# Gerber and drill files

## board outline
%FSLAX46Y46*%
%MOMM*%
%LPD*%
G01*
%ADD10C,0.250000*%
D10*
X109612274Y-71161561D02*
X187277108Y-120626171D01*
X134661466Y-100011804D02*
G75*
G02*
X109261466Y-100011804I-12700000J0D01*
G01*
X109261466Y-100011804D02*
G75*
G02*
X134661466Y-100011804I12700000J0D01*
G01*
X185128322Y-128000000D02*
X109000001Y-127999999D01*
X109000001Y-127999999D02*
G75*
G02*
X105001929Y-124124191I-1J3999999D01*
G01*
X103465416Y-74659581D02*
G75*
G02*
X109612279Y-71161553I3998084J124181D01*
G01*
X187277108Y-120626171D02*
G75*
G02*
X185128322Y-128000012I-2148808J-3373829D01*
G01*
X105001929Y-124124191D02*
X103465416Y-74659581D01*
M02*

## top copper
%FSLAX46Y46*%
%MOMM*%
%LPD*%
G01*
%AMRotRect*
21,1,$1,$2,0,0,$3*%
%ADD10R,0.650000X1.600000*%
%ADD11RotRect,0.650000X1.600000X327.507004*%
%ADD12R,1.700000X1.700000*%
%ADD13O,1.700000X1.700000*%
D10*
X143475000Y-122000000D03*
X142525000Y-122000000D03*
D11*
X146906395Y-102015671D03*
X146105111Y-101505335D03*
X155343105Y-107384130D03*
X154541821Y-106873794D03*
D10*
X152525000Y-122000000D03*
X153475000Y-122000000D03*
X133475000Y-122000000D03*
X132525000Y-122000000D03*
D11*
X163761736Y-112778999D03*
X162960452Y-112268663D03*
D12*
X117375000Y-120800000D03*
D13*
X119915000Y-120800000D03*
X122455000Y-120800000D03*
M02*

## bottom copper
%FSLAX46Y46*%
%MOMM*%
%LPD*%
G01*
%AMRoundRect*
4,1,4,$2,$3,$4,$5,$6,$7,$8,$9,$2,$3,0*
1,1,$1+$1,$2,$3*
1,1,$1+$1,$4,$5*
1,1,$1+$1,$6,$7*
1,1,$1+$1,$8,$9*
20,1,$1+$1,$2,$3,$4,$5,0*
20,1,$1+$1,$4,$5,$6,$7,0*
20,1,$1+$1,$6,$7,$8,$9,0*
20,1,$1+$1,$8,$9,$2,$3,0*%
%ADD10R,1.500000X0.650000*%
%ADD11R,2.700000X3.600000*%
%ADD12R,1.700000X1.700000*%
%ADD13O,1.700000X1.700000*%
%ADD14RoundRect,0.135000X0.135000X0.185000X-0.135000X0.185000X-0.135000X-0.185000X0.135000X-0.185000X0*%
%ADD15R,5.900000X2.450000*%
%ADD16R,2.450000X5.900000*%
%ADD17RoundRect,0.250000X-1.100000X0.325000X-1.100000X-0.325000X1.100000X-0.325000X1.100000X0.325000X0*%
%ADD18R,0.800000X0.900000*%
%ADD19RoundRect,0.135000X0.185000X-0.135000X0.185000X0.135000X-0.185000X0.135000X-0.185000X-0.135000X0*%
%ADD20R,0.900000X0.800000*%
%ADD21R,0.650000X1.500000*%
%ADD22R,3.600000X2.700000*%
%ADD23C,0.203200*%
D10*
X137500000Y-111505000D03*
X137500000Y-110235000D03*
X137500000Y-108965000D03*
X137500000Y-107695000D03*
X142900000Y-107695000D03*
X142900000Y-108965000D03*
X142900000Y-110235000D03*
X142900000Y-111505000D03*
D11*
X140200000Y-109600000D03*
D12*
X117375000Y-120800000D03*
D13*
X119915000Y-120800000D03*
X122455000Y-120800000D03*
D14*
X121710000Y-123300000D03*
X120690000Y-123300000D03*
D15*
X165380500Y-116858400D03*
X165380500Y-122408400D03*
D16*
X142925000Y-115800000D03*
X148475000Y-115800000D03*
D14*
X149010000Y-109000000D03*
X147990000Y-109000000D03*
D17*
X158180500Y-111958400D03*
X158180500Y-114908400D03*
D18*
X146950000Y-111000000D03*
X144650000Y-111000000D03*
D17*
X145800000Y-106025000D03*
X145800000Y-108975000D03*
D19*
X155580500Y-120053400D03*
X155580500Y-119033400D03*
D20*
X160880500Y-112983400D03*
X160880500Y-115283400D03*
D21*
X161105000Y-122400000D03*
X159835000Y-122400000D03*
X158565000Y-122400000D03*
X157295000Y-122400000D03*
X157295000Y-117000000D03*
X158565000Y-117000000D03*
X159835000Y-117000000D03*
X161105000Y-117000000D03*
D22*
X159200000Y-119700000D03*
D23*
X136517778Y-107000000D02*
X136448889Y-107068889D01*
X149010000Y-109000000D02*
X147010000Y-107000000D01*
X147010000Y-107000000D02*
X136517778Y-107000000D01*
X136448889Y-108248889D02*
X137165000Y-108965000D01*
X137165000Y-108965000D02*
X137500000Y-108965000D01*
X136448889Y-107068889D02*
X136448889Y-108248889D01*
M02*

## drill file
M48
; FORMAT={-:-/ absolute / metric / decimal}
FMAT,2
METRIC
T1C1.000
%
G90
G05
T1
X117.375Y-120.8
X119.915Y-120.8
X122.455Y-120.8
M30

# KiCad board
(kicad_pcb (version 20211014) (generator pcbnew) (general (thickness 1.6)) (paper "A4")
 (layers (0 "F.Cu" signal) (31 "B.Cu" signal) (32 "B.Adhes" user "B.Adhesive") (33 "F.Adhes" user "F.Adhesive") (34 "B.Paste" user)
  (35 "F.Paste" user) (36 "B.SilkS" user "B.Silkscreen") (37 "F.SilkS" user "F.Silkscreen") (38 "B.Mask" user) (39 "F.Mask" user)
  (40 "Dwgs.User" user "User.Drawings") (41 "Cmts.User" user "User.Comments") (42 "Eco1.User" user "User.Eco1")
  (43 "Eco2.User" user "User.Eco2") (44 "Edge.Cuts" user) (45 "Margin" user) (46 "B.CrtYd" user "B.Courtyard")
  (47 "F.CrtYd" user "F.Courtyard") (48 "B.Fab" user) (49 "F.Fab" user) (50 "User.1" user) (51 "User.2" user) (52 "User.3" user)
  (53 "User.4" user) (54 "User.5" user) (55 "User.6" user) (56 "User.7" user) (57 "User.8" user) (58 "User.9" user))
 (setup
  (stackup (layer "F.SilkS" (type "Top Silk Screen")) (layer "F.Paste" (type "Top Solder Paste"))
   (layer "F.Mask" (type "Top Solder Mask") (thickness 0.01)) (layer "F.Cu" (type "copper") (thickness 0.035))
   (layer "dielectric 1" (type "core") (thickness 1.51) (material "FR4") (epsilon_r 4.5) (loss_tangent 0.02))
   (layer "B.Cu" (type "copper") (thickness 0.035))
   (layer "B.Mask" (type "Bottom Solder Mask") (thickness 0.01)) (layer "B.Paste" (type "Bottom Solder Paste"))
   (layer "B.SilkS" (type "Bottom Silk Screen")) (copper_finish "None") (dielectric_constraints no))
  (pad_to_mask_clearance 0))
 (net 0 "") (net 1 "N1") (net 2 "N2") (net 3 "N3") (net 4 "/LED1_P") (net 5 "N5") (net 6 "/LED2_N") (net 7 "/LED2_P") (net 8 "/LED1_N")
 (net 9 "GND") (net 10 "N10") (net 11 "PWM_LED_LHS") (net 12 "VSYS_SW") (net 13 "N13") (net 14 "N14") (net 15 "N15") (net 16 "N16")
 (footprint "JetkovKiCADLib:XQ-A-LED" (layer "F.Cu") (at 143 122)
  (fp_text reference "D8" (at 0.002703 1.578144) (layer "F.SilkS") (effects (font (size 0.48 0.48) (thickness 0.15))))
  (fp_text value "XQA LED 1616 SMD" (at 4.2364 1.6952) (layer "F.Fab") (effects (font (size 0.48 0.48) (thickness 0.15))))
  (pad "1" smd rect (at 0.475 0) (size 0.65 1.6) (layers "F.Cu" "F.Paste" "F.Mask") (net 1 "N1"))
  (pad "2" smd rect (at -0.475 0) (size 0.65 1.6) (layers "F.Cu" "F.Paste" "F.Mask") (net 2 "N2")))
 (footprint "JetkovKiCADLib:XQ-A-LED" (layer "F.Cu") (at 146.505753 101.760503 -32.49299601)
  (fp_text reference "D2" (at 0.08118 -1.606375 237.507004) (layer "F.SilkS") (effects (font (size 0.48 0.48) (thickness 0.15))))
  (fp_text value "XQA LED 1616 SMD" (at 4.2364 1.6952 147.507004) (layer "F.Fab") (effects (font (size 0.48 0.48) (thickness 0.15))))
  (pad "1" smd rect (at 0.475 0 327.507004) (size 0.65 1.6) (layers "F.Cu" "F.Paste" "F.Mask") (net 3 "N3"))
  (pad "2" smd rect (at -0.475 0 327.507004) (size 0.65 1.6) (layers "F.Cu" "F.Paste" "F.Mask") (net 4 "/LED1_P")))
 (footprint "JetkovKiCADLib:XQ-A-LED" (layer "F.Cu") (at 154.942463 107.128962 -32.49299601)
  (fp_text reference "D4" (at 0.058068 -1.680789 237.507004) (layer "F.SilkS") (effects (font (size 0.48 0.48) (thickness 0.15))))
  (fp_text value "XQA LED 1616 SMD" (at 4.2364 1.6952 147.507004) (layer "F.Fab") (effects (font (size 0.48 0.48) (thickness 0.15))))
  (pad "1" smd rect (at 0.475 0 327.507004) (size 0.65 1.6) (layers "F.Cu" "F.Paste" "F.Mask") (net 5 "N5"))
  (pad "2" smd rect (at -0.475 0 327.507004) (size 0.65 1.6) (layers "F.Cu" "F.Paste" "F.Mask") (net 3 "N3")))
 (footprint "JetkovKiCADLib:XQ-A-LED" (layer "F.Cu") (at 153 122 180)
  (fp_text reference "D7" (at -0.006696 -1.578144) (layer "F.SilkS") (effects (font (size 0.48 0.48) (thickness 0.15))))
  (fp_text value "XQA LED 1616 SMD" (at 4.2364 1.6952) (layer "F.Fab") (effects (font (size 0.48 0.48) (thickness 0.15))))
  (pad "1" smd rect (at 0.475 0 180) (size 0.65 1.6) (layers "F.Cu" "F.Paste" "F.Mask") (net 1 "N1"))
  (pad "2" smd rect (at -0.475 0 180) (size 0.65 1.6) (layers "F.Cu" "F.Paste" "F.Mask") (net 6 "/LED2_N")))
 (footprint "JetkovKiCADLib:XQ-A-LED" (layer "F.Cu") (at 133 122)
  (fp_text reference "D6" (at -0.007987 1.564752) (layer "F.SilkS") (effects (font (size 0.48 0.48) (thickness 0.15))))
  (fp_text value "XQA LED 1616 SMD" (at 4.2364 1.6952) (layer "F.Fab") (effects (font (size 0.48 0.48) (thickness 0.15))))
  (pad "1" smd rect (at 0.475 0) (size 0.65 1.6) (layers "F.Cu" "F.Paste" "F.Mask") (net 2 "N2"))
  (pad "2" smd rect (at -0.475 0) (size 0.65 1.6) (layers "F.Cu" "F.Paste" "F.Mask") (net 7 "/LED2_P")))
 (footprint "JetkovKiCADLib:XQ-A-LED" (layer "F.Cu") (at 163.361094 112.523831 -32.49299601)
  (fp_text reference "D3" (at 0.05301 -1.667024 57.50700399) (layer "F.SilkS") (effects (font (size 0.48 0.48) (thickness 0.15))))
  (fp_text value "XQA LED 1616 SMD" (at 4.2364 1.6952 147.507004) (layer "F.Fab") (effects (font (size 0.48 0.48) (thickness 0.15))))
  (pad "1" smd rect (at 0.475 0 327.507004) (size 0.65 1.6) (layers "F.Cu" "F.Paste" "F.Mask") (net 5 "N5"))
  (pad "2" smd rect (at -0.475 0 327.507004) (size 0.65 1.6) (layers "F.Cu" "F.Paste" "F.Mask") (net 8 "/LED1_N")))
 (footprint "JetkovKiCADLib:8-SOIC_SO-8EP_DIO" (layer "B.Cu") (at 140.2 109.6)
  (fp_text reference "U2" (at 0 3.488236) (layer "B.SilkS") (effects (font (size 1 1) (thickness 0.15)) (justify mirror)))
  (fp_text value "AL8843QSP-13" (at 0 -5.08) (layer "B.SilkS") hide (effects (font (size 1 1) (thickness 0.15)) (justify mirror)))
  (pad "1" smd rect (at -2.7 1.905) (size 1.5 0.65) (layers "B.Cu" "B.Paste" "B.Mask") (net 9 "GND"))
  (pad "2" smd rect (at -2.7 0.635) (size 1.5 0.65) (layers "B.Cu" "B.Paste" "B.Mask") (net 9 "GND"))
  (pad "3" smd rect (at -2.7 -0.635) (size 1.5 0.65) (layers "B.Cu" "B.Paste" "B.Mask") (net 7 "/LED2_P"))
  (pad "4" smd rect (at -2.7 -1.905) (size 1.5 0.65) (layers "B.Cu" "B.Paste" "B.Mask") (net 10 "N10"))
  (pad "5" smd rect (at 2.7 -1.905) (size 1.5 0.65) (layers "B.Cu" "B.Paste" "B.Mask") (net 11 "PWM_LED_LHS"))
  (pad "6" smd rect (at 2.7 -0.635) (size 1.5 0.65) (layers "B.Cu" "B.Paste" "B.Mask") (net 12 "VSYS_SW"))
  (pad "7" smd rect (at 2.7 0.635) (size 1.5 0.65) (layers "B.Cu" "B.Paste" "B.Mask") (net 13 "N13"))
  (pad "8" smd rect (at 2.7 1.905) (size 1.5 0.65) (layers "B.Cu" "B.Paste" "B.Mask") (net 13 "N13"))
  (pad "EPAD" smd rect (at 0 0) (size 2.7 3.6) (layers "B.Cu" "B.Mask") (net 9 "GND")))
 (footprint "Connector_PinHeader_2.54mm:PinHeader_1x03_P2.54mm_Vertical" (layer "B.Cu") (at 117.375 120.8 -90)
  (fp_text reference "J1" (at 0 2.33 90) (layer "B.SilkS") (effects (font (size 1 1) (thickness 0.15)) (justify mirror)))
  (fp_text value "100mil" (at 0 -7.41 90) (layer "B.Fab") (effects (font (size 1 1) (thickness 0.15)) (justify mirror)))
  (pad "1" thru_hole rect locked (at 0 0 270) (size 1.7 1.7) (drill 1) (layers *.Cu *.Mask) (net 12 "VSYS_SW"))
  (pad "2" thru_hole oval locked (at 0 -2.54 270) (size 1.7 1.7) (drill 1) (layers *.Cu *.Mask) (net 11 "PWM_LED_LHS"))
  (pad "3" thru_hole oval locked (at 0 -5.08 270) (size 1.7 1.7) (drill 1) (layers *.Cu *.Mask) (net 9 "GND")))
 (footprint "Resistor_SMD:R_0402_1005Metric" (layer "B.Cu") (at 121.2 123.3 180)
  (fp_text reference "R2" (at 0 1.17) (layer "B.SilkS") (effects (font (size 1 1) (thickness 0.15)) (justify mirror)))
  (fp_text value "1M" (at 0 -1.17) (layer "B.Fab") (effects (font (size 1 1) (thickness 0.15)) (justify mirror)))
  (pad "1" smd roundrect locked (at -0.51 0 180) (size 0.54 0.64) (layers "B.Cu" "B.Paste" "B.Mask") (roundrect_rratio 0.25) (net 9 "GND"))
  (pad "2" smd roundrect locked (at 0.51 0 180) (size 0.54 0.64) (layers "B.Cu" "B.Paste" "B.Mask") (roundrect_rratio 0.25)
   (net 11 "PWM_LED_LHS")))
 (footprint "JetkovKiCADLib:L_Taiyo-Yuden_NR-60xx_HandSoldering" (layer "B.Cu") (at 165.3805 119.6334 -90)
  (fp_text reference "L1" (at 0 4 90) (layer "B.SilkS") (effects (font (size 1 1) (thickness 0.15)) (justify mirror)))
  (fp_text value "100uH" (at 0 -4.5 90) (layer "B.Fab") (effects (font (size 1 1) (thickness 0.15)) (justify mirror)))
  (pad "1" smd rect (at -2.775 0 270) (size 2.45 5.9) (layers "B.Cu" "B.Paste" "B.Mask") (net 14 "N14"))
  (pad "2" smd rect (at 2.775 0 270) (size 2.45 5.9) (layers "B.Cu" "B.Paste" "B.Mask") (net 8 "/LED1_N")))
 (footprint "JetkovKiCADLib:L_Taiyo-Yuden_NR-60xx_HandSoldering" (layer "B.Cu") (at 145.7 115.8)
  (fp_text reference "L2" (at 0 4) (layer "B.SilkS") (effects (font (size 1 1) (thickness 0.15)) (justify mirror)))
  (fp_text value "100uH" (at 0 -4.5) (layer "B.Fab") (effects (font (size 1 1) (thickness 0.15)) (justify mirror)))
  (pad "1" smd rect (at -2.775 0) (size 2.45 5.9) (layers "B.Cu" "B.Paste" "B.Mask") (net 13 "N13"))
  (pad "2" smd rect (at 2.775 0) (size 2.45 5.9) (layers "B.Cu" "B.Paste" "B.Mask") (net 6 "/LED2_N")))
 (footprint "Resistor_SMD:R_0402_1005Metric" (layer "B.Cu") (at 148.5 109 180)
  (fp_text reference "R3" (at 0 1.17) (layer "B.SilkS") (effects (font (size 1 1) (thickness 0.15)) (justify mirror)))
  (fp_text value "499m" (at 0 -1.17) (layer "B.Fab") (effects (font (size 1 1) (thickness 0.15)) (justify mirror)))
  (pad "1" smd roundrect locked (at -0.51 0 180) (size 0.54 0.64) (layers "B.Cu" "B.Paste" "B.Mask") (roundrect_rratio 0.25)
   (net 7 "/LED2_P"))
  (pad "2" smd roundrect locked (at 0.51 0 180) (size 0.54 0.64) (layers "B.Cu" "B.Paste" "B.Mask") (roundrect_rratio 0.25)
   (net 12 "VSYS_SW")))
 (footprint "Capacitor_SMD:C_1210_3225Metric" (layer "B.Cu") (at 158.1805 113.4334 -90)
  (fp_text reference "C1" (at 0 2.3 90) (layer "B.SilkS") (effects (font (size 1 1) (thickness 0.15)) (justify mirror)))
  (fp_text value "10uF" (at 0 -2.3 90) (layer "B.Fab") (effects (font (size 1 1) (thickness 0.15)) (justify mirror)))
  (pad "1" smd roundrect locked (at -1.475 0 270) (size 1.15 2.7) (layers "B.Cu" "B.Paste" "B.Mask") (roundrect_rratio 0.217391)
   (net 9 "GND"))
  (pad "2" smd roundrect locked (at 1.475 0 270) (size 1.15 2.7) (layers "B.Cu" "B.Paste" "B.Mask") (roundrect_rratio 0.217391)
   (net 12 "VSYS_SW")))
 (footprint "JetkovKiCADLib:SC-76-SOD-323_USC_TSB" (layer "B.Cu") (at 145.8 111 180)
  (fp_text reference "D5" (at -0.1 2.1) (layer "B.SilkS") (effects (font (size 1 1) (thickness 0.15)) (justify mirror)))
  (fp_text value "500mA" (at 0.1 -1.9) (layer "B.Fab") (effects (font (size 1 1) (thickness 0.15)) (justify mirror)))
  (pad "1" smd rect (at -1.15 0 180) (size 0.8 0.9) (layers "B.Cu" "B.Paste" "B.Mask") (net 12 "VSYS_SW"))
  (pad "2" smd rect (at 1.15 0 180) (size 0.8 0.9) (layers "B.Cu" "B.Paste" "B.Mask") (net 13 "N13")))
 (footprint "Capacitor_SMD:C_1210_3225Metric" (layer "B.Cu") (at 145.8 107.5 -90)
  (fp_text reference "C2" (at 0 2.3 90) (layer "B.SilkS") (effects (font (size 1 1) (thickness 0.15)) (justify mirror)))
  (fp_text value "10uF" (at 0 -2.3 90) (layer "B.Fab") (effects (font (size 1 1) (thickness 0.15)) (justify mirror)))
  (pad "1" smd roundrect locked (at -1.475 0 270) (size 1.15 2.7) (layers "B.Cu" "B.Paste" "B.Mask") (roundrect_rratio 0.217391)
   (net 9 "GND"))
  (pad "2" smd roundrect locked (at 1.475 0 270) (size 1.15 2.7) (layers "B.Cu" "B.Paste" "B.Mask") (roundrect_rratio 0.217391)
   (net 12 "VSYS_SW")))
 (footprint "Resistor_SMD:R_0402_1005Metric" (layer "B.Cu") (at 155.5805 119.5434 90)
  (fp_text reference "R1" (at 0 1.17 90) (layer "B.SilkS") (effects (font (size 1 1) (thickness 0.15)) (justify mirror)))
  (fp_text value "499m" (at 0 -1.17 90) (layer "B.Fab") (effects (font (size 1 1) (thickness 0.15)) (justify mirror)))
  (pad "1" smd roundrect locked (at -0.51 0 90) (size 0.54 0.64) (layers "B.Cu" "B.Paste" "B.Mask") (roundrect_rratio 0.25)
   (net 4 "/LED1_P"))
  (pad "2" smd roundrect locked (at 0.51 0 90) (size 0.54 0.64) (layers "B.Cu" "B.Paste" "B.Mask") (roundrect_rratio 0.25)
   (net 12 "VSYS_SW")))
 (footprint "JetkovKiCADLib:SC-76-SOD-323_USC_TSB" (layer "B.Cu") (at 160.8805 114.1334 -90)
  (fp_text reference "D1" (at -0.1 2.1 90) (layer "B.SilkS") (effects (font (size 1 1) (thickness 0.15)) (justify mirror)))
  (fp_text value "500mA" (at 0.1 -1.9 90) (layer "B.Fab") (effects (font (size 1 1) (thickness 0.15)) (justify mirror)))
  (pad "1" smd rect (at -1.15 0 270) (size 0.8 0.9) (layers "B.Cu" "B.Paste" "B.Mask") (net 12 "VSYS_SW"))
  (pad "2" smd rect (at 1.15 0 270) (size 0.8 0.9) (layers "B.Cu" "B.Paste" "B.Mask") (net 14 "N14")))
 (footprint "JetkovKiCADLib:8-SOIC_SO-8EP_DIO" (layer "B.Cu") (at 159.2 119.7 90)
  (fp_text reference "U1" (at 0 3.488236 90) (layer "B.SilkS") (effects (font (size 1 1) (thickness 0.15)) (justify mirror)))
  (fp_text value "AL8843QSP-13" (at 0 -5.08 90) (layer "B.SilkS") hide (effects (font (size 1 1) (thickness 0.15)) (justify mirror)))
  (pad "1" smd rect (at -2.7 1.905 90) (size 1.5 0.65) (layers "B.Cu" "B.Paste" "B.Mask") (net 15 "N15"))
  (pad "2" smd rect (at -2.7 0.635 90) (size 1.5 0.65) (layers "B.Cu" "B.Paste" "B.Mask") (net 15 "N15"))
  (pad "3" smd rect (at -2.7 -0.635 90) (size 1.5 0.65) (layers "B.Cu" "B.Paste" "B.Mask") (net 4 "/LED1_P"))
  (pad "4" smd rect (at -2.7 -1.905 90) (size 1.5 0.65) (layers "B.Cu" "B.Paste" "B.Mask") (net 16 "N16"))
  (pad "5" smd rect (at 2.7 -1.905 90) (size 1.5 0.65) (layers "B.Cu" "B.Paste" "B.Mask") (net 11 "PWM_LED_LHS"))
  (pad "6" smd rect (at 2.7 -0.635 90) (size 1.5 0.65) (layers "B.Cu" "B.Paste" "B.Mask") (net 12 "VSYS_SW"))
  (pad "7" smd rect (at 2.7 0.635 90) (size 1.5 0.65) (layers "B.Cu" "B.Paste" "B.Mask") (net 14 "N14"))
  (pad "8" smd rect (at 2.7 1.905 90) (size 1.5 0.65) (layers "B.Cu" "B.Paste" "B.Mask") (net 14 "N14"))
  (pad "EPAD" smd rect (at 0 0 90) (size 2.7 3.6) (layers "B.Cu" "B.Mask") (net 15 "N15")))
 (gr_line locked (start 109.612274 71.161561) (end 187.277108 120.626171) (layer "Edge.Cuts") (width 0.25))
 (gr_circle locked (center 121.961466 100.011804) (end 131.180191 108.747084) (layer "Edge.Cuts") (width 0.25) (fill none))
 (gr_line locked (start 185.128322 128) (end 109.000001 127.999999) (layer "Edge.Cuts") (width 0.25))
 (gr_arc locked (start 109.000001 127.999999) (mid 106.215829 126.871999) (end 105.001929 124.124191) (layer "Edge.Cuts") (width 0.25))
 (gr_arc locked (start 103.465416 74.659581) (mid 105.485105 71.058898) (end 109.612274 71.161561) (layer "Edge.Cuts") (width 0.25))
 (gr_arc locked (start 187.277108 120.626171) (mid 188.96859 125.119081) (end 185.128322 128) (layer "Edge.Cuts") (width 0.25))
 (gr_line locked (start 105.001929 124.124191) (end 103.465416 74.659581) (layer "Edge.Cuts") (width 0.25))
 (segment (start 136.517778 107) (end 136.448889 107.068889) (width 0.2032) (layer "B.Cu") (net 7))
 (segment (start 149.01 109) (end 147.01 107) (width 0.2032) (layer "B.Cu") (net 7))
 (segment (start 147.01 107) (end 136.517778 107) (width 0.2032) (layer "B.Cu") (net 7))
 (segment (start 136.448889 108.248889) (end 137.165 108.965) (width 0.2032) (layer "B.Cu") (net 7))
 (segment (start 137.165 108.965) (end 137.5 108.965) (width 0.2032) (layer "B.Cu") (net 7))
 (segment (start 136.448889 107.068889) (end 136.448889 108.248889) (width 0.2032) (layer "B.Cu") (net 7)))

